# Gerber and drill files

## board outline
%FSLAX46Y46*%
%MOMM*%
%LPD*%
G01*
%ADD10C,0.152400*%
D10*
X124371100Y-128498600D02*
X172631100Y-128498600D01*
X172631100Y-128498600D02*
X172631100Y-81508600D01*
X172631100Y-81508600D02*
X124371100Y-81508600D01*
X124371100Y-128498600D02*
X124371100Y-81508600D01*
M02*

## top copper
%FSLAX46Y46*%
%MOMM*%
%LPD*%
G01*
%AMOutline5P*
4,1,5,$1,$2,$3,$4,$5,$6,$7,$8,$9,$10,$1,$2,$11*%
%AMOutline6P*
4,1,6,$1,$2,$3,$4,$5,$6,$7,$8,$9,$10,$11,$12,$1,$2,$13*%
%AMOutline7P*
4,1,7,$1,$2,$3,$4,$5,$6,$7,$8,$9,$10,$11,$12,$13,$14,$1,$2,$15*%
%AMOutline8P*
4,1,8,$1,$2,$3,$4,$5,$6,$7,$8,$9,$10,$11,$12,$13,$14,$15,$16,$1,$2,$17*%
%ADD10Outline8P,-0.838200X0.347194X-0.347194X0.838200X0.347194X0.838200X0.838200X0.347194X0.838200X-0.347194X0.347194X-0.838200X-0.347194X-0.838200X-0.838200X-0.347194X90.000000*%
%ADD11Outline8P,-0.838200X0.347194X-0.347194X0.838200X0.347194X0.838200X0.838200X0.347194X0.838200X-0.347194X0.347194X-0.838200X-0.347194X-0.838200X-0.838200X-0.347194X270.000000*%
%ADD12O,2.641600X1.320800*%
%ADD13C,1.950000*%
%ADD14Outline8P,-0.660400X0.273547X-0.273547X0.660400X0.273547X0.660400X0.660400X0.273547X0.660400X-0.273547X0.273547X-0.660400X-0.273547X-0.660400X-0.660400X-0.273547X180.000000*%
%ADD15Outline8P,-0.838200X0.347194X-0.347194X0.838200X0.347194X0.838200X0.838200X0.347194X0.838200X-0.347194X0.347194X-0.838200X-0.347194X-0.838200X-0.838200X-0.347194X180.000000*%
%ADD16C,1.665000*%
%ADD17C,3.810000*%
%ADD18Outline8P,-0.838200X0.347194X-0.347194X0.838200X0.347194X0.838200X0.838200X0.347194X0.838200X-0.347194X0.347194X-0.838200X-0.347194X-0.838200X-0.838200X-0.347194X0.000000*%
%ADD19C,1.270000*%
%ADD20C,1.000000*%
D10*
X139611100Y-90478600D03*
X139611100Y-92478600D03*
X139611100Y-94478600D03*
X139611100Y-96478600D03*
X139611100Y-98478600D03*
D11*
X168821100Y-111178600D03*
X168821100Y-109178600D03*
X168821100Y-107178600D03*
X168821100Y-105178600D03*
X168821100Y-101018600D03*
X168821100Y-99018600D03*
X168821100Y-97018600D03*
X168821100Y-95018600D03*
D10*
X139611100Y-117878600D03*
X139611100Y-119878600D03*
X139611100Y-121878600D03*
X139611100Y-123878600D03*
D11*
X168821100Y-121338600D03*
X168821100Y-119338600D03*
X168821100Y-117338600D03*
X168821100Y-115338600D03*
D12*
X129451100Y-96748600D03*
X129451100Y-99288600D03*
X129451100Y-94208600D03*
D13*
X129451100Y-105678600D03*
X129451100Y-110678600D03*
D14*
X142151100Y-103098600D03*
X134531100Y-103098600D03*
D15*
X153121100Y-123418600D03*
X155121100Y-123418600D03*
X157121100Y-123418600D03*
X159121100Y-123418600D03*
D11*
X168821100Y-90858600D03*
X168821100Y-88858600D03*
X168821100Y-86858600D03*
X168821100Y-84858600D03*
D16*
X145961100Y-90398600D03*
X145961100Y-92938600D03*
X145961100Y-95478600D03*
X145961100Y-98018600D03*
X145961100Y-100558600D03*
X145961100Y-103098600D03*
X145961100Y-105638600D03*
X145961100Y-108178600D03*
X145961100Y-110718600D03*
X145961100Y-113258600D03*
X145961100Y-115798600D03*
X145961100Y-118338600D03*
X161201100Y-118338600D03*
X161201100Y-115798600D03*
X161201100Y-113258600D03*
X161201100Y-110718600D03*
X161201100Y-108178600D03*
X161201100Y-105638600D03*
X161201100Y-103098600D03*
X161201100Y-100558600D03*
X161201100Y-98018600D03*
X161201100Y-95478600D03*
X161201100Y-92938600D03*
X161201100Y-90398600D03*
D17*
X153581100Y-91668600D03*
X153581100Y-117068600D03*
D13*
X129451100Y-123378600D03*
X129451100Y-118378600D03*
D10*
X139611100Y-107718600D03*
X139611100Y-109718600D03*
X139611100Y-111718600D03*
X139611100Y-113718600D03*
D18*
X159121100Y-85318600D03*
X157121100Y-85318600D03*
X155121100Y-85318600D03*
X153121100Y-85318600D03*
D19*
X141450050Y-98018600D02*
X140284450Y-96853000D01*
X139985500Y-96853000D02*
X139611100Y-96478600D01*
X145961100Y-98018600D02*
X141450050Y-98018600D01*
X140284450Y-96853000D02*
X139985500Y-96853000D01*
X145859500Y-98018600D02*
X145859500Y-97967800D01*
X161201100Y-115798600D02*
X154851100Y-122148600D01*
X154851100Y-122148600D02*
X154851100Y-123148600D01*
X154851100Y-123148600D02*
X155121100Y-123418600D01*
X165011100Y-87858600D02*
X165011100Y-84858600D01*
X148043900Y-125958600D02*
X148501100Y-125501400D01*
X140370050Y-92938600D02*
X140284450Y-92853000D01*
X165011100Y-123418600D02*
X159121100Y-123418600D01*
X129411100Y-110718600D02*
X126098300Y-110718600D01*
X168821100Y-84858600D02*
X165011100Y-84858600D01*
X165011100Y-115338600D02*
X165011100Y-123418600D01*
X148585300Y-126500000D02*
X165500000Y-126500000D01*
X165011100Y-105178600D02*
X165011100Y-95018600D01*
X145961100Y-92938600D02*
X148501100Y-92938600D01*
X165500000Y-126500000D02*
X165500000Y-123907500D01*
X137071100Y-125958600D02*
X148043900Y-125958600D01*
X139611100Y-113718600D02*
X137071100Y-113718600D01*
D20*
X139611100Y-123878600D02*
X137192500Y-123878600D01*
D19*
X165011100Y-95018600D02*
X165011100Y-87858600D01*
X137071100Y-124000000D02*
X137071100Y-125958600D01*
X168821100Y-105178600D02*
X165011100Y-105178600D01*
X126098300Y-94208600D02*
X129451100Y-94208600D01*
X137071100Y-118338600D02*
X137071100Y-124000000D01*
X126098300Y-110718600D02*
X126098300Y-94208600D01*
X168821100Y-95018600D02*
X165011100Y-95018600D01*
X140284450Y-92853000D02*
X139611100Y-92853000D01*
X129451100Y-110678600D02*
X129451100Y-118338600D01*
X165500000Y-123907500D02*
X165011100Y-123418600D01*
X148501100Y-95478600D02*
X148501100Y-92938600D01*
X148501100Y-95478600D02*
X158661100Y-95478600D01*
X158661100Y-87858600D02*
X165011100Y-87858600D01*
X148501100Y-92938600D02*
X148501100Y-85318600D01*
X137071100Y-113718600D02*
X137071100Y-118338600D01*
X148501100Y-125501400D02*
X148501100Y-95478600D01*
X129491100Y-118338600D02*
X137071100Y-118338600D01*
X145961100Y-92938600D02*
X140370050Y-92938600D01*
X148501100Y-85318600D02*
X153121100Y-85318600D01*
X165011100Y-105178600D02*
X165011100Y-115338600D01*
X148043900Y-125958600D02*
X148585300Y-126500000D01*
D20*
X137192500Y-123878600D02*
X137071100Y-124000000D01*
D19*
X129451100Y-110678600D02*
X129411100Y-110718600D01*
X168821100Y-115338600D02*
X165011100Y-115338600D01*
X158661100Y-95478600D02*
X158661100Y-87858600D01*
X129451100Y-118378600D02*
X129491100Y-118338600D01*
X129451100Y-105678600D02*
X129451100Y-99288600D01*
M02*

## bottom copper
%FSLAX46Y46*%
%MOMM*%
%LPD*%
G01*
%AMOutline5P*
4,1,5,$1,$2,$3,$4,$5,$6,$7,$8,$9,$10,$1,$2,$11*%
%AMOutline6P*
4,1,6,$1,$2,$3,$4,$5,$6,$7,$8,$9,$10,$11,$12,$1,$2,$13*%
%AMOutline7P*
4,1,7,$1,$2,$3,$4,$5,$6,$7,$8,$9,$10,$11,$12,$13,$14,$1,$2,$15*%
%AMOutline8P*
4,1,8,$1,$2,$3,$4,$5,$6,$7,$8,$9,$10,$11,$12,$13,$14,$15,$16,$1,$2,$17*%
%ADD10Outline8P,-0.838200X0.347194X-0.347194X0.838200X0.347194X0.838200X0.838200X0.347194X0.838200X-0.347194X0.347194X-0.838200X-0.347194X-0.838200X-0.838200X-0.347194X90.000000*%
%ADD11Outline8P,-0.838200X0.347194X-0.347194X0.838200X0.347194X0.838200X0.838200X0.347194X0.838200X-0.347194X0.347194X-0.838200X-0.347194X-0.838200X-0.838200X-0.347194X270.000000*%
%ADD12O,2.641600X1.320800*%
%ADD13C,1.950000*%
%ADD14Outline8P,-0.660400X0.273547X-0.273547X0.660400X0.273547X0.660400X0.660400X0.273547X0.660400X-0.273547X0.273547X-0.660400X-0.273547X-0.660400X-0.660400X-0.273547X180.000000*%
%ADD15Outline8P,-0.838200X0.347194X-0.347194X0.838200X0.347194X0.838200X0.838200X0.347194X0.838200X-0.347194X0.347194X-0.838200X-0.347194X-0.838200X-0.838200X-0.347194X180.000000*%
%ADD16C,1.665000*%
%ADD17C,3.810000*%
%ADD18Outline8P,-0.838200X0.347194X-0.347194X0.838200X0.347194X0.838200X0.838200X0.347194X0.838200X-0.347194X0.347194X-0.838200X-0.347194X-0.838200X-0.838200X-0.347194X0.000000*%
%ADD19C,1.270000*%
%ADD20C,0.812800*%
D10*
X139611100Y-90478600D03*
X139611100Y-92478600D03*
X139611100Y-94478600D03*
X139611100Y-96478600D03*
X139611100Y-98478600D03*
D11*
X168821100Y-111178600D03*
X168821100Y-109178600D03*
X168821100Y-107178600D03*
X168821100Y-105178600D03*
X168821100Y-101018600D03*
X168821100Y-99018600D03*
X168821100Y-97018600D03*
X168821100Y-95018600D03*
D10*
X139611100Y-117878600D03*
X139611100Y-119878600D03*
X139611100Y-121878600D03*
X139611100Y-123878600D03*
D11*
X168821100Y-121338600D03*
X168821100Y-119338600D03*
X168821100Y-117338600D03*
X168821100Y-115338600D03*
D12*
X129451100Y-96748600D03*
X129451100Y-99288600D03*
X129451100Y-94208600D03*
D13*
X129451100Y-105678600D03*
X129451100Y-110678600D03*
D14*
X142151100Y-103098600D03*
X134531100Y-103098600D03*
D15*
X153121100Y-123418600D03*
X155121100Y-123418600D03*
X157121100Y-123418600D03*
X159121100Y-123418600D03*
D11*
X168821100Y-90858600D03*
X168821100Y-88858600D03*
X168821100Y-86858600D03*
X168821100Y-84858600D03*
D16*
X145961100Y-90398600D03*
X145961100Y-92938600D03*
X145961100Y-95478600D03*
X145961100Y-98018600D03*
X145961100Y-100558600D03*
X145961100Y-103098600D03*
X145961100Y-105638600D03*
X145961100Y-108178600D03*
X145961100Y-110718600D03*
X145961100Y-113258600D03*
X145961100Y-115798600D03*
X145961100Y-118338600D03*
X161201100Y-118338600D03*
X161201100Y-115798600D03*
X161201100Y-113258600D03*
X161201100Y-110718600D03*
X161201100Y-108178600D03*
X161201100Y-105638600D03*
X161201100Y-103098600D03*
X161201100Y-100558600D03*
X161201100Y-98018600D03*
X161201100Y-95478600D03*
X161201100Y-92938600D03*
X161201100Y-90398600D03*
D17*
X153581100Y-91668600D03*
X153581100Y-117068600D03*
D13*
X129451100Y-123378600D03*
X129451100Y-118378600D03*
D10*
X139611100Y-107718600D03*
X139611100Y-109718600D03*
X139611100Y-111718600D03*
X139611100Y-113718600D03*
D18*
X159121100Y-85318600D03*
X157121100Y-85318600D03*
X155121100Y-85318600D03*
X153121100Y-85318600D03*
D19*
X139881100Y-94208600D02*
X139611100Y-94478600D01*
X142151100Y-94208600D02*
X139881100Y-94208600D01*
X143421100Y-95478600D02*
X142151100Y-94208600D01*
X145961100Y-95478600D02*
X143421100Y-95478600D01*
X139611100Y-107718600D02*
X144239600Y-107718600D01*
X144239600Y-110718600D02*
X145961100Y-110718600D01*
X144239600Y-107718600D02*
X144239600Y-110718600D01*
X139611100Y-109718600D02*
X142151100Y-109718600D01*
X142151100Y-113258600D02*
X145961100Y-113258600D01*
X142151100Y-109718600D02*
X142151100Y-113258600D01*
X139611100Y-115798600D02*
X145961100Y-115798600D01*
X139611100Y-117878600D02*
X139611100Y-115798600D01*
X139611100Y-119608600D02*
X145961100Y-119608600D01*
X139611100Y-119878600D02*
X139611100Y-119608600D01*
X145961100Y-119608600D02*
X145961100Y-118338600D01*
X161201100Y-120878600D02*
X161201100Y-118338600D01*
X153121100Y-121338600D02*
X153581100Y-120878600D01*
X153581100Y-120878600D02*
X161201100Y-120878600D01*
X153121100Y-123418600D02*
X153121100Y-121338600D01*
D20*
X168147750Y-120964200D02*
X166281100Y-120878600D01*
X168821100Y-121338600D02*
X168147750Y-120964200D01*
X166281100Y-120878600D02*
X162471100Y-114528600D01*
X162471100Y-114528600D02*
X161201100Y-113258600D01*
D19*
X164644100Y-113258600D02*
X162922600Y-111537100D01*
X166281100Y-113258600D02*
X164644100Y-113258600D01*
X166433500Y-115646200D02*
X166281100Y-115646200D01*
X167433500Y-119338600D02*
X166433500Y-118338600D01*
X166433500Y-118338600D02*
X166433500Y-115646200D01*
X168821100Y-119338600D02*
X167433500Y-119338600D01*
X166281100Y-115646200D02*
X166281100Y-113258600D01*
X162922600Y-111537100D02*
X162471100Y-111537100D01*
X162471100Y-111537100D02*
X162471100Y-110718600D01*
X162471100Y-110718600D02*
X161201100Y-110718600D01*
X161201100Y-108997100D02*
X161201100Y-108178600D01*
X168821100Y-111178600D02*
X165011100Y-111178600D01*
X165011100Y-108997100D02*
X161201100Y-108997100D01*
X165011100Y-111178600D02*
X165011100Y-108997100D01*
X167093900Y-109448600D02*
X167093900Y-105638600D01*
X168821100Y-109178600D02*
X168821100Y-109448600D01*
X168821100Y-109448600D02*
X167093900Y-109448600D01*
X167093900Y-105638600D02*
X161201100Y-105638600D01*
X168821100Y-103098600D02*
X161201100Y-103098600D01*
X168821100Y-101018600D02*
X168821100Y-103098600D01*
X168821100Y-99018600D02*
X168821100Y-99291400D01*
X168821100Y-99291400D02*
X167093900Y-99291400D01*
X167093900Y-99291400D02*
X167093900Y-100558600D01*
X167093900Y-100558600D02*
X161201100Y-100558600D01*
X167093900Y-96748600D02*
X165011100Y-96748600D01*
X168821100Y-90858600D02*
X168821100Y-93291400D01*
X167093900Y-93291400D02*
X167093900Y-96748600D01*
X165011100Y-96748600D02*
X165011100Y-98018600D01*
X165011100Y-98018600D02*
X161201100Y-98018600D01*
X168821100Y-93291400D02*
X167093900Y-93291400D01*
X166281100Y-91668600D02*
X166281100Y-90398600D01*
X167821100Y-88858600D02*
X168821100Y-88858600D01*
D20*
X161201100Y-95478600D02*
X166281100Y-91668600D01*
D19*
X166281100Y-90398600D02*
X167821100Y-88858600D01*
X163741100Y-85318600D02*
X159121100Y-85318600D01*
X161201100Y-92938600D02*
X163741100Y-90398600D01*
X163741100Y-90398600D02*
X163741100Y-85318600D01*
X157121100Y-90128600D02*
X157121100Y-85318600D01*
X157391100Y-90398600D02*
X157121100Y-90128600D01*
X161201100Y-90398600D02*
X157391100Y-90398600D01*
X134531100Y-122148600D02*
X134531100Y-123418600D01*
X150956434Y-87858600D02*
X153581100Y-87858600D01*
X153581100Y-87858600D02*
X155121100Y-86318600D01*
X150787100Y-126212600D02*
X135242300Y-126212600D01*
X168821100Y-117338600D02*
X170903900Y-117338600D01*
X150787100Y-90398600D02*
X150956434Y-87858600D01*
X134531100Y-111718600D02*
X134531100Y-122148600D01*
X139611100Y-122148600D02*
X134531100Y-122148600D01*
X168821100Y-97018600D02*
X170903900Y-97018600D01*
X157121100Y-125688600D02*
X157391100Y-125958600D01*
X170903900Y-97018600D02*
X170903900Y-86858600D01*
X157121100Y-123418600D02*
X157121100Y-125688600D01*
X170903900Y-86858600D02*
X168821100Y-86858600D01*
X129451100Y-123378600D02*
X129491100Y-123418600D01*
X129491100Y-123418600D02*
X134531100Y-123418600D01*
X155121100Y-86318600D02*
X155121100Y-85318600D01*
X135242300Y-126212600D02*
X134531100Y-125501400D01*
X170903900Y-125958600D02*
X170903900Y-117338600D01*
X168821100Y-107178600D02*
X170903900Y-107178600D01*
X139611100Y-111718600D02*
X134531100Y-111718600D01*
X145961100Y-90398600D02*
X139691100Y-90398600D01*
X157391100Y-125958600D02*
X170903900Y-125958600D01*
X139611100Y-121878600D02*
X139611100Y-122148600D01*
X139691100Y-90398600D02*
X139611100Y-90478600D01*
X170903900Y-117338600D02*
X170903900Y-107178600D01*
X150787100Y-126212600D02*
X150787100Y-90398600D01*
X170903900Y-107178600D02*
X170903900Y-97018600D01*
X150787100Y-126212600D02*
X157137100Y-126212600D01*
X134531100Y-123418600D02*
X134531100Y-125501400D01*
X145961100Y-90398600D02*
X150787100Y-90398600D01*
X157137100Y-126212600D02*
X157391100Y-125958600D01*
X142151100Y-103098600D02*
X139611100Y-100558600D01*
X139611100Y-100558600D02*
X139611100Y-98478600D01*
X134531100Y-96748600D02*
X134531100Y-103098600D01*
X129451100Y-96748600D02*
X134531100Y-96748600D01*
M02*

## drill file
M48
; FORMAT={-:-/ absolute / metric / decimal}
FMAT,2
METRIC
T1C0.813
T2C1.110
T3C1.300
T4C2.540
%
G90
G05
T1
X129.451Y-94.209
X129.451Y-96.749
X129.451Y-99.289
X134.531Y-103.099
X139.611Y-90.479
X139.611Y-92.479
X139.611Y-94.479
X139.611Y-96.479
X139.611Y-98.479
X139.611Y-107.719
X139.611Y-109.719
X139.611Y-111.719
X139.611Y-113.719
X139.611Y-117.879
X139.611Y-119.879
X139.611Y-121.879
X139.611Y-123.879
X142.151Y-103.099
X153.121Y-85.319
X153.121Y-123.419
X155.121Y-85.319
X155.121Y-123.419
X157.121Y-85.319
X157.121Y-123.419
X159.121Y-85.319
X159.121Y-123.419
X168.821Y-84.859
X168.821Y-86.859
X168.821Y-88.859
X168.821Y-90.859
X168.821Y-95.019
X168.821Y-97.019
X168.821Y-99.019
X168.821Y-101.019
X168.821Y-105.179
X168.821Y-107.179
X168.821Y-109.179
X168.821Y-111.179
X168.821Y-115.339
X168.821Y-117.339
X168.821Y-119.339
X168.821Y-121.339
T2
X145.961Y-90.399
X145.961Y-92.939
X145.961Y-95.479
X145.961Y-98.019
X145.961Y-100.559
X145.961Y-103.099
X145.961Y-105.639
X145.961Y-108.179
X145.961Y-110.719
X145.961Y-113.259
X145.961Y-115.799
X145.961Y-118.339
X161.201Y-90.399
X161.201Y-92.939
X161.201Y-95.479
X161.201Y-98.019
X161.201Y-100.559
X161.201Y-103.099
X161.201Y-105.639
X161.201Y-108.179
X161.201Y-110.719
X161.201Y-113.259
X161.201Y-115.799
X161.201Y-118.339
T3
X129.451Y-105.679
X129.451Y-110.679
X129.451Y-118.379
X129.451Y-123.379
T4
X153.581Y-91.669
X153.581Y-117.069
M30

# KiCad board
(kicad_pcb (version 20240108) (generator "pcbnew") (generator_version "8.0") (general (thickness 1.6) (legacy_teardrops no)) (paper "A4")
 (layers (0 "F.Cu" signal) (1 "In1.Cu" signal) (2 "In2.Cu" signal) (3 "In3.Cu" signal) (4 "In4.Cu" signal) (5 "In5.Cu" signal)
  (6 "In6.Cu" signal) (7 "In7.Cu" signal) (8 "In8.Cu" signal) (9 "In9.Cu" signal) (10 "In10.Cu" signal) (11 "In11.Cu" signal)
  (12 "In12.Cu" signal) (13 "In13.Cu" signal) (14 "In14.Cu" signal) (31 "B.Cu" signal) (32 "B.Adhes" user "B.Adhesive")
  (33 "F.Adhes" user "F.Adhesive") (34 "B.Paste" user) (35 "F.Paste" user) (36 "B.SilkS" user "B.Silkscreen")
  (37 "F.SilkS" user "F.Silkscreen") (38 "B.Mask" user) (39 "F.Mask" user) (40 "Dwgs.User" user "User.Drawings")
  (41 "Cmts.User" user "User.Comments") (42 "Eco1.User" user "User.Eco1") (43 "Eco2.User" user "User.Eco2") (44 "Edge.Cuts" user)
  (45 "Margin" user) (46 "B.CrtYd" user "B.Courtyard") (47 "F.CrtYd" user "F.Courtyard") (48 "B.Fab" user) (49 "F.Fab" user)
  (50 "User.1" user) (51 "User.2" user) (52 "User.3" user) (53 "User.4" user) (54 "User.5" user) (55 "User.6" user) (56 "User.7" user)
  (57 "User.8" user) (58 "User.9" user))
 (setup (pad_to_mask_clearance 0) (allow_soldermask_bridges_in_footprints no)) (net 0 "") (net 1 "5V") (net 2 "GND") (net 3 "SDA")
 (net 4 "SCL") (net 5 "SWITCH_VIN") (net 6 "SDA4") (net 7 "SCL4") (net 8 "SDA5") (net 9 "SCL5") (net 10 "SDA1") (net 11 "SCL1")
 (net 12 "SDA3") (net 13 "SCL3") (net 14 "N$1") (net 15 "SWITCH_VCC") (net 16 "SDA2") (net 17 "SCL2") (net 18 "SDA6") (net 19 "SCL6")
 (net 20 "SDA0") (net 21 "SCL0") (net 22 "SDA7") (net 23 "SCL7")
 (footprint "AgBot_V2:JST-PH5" (layer "F.Cu") (at 139.6111 95.4786 90)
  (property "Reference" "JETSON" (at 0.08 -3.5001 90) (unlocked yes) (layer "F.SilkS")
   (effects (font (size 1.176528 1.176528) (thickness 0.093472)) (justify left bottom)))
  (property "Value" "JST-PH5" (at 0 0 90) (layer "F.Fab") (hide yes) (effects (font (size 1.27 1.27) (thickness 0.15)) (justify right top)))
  (pad "1" thru_hole roundrect (at 5 0 90) (size 1.6764 1.6764) (drill 0.8128) (layers "*.Cu" "*.Mask") (remove_unused_layers no)
   (roundrect_rratio 0.25) (chamfer_ratio 0.2928932188) (chamfer top_left top_right bottom_left bottom_right) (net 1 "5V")
   (solder_mask_margin 0.1016) (thermal_bridge_angle 0))
  (pad "2" thru_hole roundrect (at 3 0 90) (size 1.6764 1.6764) (drill 0.8128) (layers "*.Cu" "*.Mask") (remove_unused_layers no)
   (roundrect_rratio 0.25) (chamfer_ratio 0.2928932188) (chamfer top_left top_right bottom_left bottom_right) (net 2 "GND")
   (solder_mask_margin 0.1016) (thermal_bridge_angle 0))
  (pad "3" thru_hole roundrect (at 1 0 90) (size 1.6764 1.6764) (drill 0.8128) (layers "*.Cu" "*.Mask") (remove_unused_layers no)
   (roundrect_rratio 0.25) (chamfer_ratio 0.2928932188) (chamfer top_left top_right bottom_left bottom_right) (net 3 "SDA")
   (solder_mask_margin 0.1016) (thermal_bridge_angle 0))
  (pad "4" thru_hole roundrect (at -1 0 90) (size 1.6764 1.6764) (drill 0.8128) (layers "*.Cu" "*.Mask") (remove_unused_layers no)
   (roundrect_rratio 0.25) (chamfer_ratio 0.2928932188) (chamfer top_left top_right bottom_left bottom_right) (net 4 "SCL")
   (solder_mask_margin 0.1016) (thermal_bridge_angle 0))
  (pad "5" thru_hole roundrect (at -3 0 90) (size 1.6764 1.6764) (drill 0.8128) (layers "*.Cu" "*.Mask") (remove_unused_layers no)
   (roundrect_rratio 0.25) (chamfer_ratio 0.2928932188) (chamfer top_left top_right bottom_left bottom_right) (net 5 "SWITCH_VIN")
   (solder_mask_margin 0.1016) (thermal_bridge_angle 0)))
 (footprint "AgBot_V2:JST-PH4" (layer "F.Cu") (at 168.8211 108.1786 -90)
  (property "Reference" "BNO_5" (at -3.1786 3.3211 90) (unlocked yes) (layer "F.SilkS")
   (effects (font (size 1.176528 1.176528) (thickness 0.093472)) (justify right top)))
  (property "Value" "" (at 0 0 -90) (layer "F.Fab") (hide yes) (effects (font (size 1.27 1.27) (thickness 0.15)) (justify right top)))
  (pad "1" thru_hole roundrect (at 3 0 270) (size 1.6764 1.6764) (drill 0.8128) (layers "*.Cu" "*.Mask") (remove_unused_layers no)
   (roundrect_rratio 0.25) (chamfer_ratio 0.2928932188) (chamfer top_left top_right bottom_left bottom_right) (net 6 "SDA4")
   (solder_mask_margin 0.1016) (thermal_bridge_angle 0))
  (pad "2" thru_hole roundrect (at 1 0 270) (size 1.6764 1.6764) (drill 0.8128) (layers "*.Cu" "*.Mask") (remove_unused_layers no)
   (roundrect_rratio 0.25) (chamfer_ratio 0.2928932188) (chamfer top_left top_right bottom_left bottom_right) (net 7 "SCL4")
   (solder_mask_margin 0.1016) (thermal_bridge_angle 0))
  (pad "3" thru_hole roundrect (at -1 0 270) (size 1.6764 1.6764) (drill 0.8128) (layers "*.Cu" "*.Mask") (remove_unused_layers no)
   (roundrect_rratio 0.25) (chamfer_ratio 0.2928932188) (chamfer top_left top_right bottom_left bottom_right) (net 1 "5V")
   (solder_mask_margin 0.1016) (thermal_bridge_angle 0))
  (pad "4" thru_hole roundrect (at -3 0 270) (size 1.6764 1.6764) (drill 0.8128) (layers "*.Cu" "*.Mask") (remove_unused_layers no)
   (roundrect_rratio 0.25) (chamfer_ratio 0.2928932188) (chamfer top_left top_right bottom_left bottom_right) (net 2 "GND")
   (solder_mask_margin 0.1016) (thermal_bridge_angle 0)))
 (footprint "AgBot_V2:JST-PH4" (layer "F.Cu") (at 168.8211 98.0186 -90)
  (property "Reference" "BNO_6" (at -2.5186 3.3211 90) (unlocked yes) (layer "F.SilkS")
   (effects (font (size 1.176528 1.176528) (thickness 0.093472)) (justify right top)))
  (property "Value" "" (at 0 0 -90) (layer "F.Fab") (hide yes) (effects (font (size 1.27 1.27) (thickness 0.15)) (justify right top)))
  (pad "1" thru_hole roundrect (at 3 0 270) (size 1.6764 1.6764) (drill 0.8128) (layers "*.Cu" "*.Mask") (remove_unused_layers no)
   (roundrect_rratio 0.25) (chamfer_ratio 0.2928932188) (chamfer top_left top_right bottom_left bottom_right) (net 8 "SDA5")
   (solder_mask_margin 0.1016) (thermal_bridge_angle 0))
  (pad "2" thru_hole roundrect (at 1 0 270) (size 1.6764 1.6764) (drill 0.8128) (layers "*.Cu" "*.Mask") (remove_unused_layers no)
   (roundrect_rratio 0.25) (chamfer_ratio 0.2928932188) (chamfer top_left top_right bottom_left bottom_right) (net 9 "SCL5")
   (solder_mask_margin 0.1016) (thermal_bridge_angle 0))
  (pad "3" thru_hole roundrect (at -1 0 270) (size 1.6764 1.6764) (drill 0.8128) (layers "*.Cu" "*.Mask") (remove_unused_layers no)
   (roundrect_rratio 0.25) (chamfer_ratio 0.2928932188) (chamfer top_left top_right bottom_left bottom_right) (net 1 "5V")
   (solder_mask_margin 0.1016) (thermal_bridge_angle 0))
  (pad "4" thru_hole roundrect (at -3 0 270) (size 1.6764 1.6764) (drill 0.8128) (layers "*.Cu" "*.Mask") (remove_unused_layers no)
   (roundrect_rratio 0.25) (chamfer_ratio 0.2928932188) (chamfer top_left top_right bottom_left bottom_right) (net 2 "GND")
   (solder_mask_margin 0.1016) (thermal_bridge_angle 0)))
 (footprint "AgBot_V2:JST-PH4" (layer "F.Cu") (at 139.6111 120.8786 90)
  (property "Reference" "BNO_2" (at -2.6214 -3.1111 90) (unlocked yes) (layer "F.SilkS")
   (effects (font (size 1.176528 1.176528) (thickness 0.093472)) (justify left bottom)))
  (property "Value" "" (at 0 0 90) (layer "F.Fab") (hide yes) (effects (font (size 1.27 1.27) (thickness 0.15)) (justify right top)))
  (pad "1" thru_hole roundrect (at 3 0 90) (size 1.6764 1.6764) (drill 0.8128) (layers "*.Cu" "*.Mask") (remove_unused_layers no)
   (roundrect_rratio 0.25) (chamfer_ratio 0.2928932188) (chamfer top_left top_right bottom_left bottom_right) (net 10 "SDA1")
   (solder_mask_margin 0.1016) (thermal_bridge_angle 0))
  (pad "2" thru_hole roundrect (at 1 0 90) (size 1.6764 1.6764) (drill 0.8128) (layers "*.Cu" "*.Mask") (remove_unused_layers no)
   (roundrect_rratio 0.25) (chamfer_ratio 0.2928932188) (chamfer top_left top_right bottom_left bottom_right) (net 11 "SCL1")
   (solder_mask_margin 0.1016) (thermal_bridge_angle 0))
  (pad "3" thru_hole roundrect (at -1 0 90) (size 1.6764 1.6764) (drill 0.8128) (layers "*.Cu" "*.Mask") (remove_unused_layers no)
   (roundrect_rratio 0.25) (chamfer_ratio 0.2928932188) (chamfer top_left top_right bottom_left bottom_right) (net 1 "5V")
   (solder_mask_margin 0.1016) (thermal_bridge_angle 0))
  (pad "4" thru_hole roundrect (at -3 0 90) (size 1.6764 1.6764) (drill 0.8128) (layers "*.Cu" "*.Mask") (remove_unused_layers no)
   (roundrect_rratio 0.25) (chamfer_ratio 0.2928932188) (chamfer top_left top_right bottom_left bottom_right) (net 2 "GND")
   (solder_mask_margin 0.1016) (thermal_bridge_angle 0)))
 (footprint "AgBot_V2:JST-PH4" (layer "F.Cu") (at 168.8211 118.3386 -90)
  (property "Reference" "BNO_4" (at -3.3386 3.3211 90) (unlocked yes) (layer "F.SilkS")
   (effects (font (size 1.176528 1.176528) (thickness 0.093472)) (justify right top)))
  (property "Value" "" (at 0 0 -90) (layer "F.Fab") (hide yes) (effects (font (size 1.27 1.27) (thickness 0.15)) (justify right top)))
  (pad "1" thru_hole roundrect (at 3 0 270) (size 1.6764 1.6764) (drill 0.8128) (layers "*.Cu" "*.Mask") (remove_unused_layers no)
   (roundrect_rratio 0.25) (chamfer_ratio 0.2928932188) (chamfer top_left top_right bottom_left bottom_right) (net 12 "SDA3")
   (solder_mask_margin 0.1016) (thermal_bridge_angle 0))
  (pad "2" thru_hole roundrect (at 1 0 270) (size 1.6764 1.6764) (drill 0.8128) (layers "*.Cu" "*.Mask") (remove_unused_layers no)
   (roundrect_rratio 0.25) (chamfer_ratio 0.2928932188) (chamfer top_left top_right bottom_left bottom_right) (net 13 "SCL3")
   (solder_mask_margin 0.1016) (thermal_bridge_angle 0))
  (pad "3" thru_hole roundrect (at -1 0 270) (size 1.6764 1.6764) (drill 0.8128) (layers "*.Cu" "*.Mask") (remove_unused_layers no)
   (roundrect_rratio 0.25) (chamfer_ratio 0.2928932188) (chamfer top_left top_right bottom_left bottom_right) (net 1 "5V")
   (solder_mask_margin 0.1016) (thermal_bridge_angle 0))
  (pad "4" thru_hole roundrect (at -3 0 270) (size 1.6764 1.6764) (drill 0.8128) (layers "*.Cu" "*.Mask") (remove_unused_layers no)
   (roundrect_rratio 0.25) (chamfer_ratio 0.2928932188) (chamfer top_left top_right bottom_left bottom_right) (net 2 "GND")
   (solder_mask_margin 0.1016) (thermal_bridge_angle 0)))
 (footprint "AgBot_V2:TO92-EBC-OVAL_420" (layer "F.Cu") (at 130.7211 96.7486 -90)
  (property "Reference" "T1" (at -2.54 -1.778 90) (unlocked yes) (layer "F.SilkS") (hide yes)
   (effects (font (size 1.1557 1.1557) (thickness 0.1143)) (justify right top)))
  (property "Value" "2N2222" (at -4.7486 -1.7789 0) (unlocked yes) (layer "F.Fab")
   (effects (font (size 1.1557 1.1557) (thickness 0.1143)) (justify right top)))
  (pad "B" thru_hole oval (at 0 1.27) (size 2.6416 1.3208) (drill 0.8128) (layers "*.Cu" "*.Mask") (remove_unused_layers no) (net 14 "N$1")
   (solder_mask_margin 0.1016) (thermal_bridge_angle 0))
  (pad "C" thru_hole oval (at 2.54 1.27) (size 2.6416 1.3208) (drill 0.8128) (layers "*.Cu" "*.Mask") (remove_unused_layers no)
   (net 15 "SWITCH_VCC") (solder_mask_margin 0.1016) (thermal_bridge_angle 0))
  (pad "E" thru_hole oval (at -2.54 1.27) (size 2.6416 1.3208) (drill 0.8128) (layers "*.Cu" "*.Mask") (remove_unused_layers no)
   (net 2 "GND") (solder_mask_margin 0.1016) (thermal_bridge_angle 0)))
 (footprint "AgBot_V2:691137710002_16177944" (layer "F.Cu") (at 129.4511 108.1786 -90)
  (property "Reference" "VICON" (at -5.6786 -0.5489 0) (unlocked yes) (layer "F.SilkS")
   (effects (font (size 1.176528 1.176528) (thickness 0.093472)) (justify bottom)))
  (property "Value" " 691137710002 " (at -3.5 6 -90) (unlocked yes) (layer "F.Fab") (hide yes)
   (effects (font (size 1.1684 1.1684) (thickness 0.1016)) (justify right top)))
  (pad "1" thru_hole circle (at -2.5 0 270) (size 1.95 1.95) (drill 1.3) (layers "*.Cu" "*.Mask") (remove_unused_layers no)
   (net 15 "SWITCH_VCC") (solder_mask_margin 0.1016) (thermal_bridge_angle 0))
  (pad "2" thru_hole circle (at 2.5 0 270) (size 1.95 1.95) (drill 1.3) (layers "*.Cu" "*.Mask") (remove_unused_layers no) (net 2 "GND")
   (solder_mask_margin 0.1016) (thermal_bridge_angle 0)))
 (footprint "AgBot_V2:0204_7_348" (layer "F.Cu") (at 138.3411 103.0986 180)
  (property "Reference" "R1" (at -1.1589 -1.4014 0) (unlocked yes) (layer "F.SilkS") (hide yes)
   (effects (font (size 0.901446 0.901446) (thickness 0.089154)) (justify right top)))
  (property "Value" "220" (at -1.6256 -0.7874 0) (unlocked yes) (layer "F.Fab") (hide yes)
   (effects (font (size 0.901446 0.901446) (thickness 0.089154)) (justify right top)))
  (pad "1" thru_hole roundrect (at -3.81 0 180) (size 1.3208 1.3208) (drill 0.8128) (layers "*.Cu" "*.Mask") (remove_unused_layers no)
   (roundrect_rratio 0.25) (chamfer_ratio 0.2928932188) (chamfer top_left top_right bottom_left bottom_right) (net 5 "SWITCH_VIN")
   (solder_mask_margin 0.1016) (thermal_bridge_angle 0))
  (pad "2" thru_hole roundrect (at 3.81 0 180) (size 1.3208 1.3208) (drill 0.8128) (layers "*.Cu" "*.Mask") (remove_unused_layers no)
   (roundrect_rratio 0.25) (chamfer_ratio 0.2928932188) (chamfer top_left top_right bottom_left bottom_right) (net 14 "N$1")
   (solder_mask_margin 0.1016) (thermal_bridge_angle 0)))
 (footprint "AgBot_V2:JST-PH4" (layer "F.Cu") (at 156.1211 123.4186 180)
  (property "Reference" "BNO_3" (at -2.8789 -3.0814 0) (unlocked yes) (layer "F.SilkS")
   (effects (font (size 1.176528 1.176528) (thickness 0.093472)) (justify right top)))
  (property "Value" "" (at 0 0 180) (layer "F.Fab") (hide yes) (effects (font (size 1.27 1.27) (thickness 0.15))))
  (pad "1" thru_hole roundrect (at 3 0 180) (size 1.6764 1.6764) (drill 0.8128) (layers "*.Cu" "*.Mask") (remove_unused_layers no)
   (roundrect_rratio 0.25) (chamfer_ratio 0.2928932188) (chamfer top_left top_right bottom_left bottom_right) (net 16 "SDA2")
   (solder_mask_margin 0.1016) (thermal_bridge_angle 0))
  (pad "2" thru_hole roundrect (at 1 0 180) (size 1.6764 1.6764) (drill 0.8128) (layers "*.Cu" "*.Mask") (remove_unused_layers no)
   (roundrect_rratio 0.25) (chamfer_ratio 0.2928932188) (chamfer top_left top_right bottom_left bottom_right) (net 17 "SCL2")
   (solder_mask_margin 0.1016) (thermal_bridge_angle 0))
  (pad "3" thru_hole roundrect (at -1 0 180) (size 1.6764 1.6764) (drill 0.8128) (layers "*.Cu" "*.Mask") (remove_unused_layers no)
   (roundrect_rratio 0.25) (chamfer_ratio 0.2928932188) (chamfer top_left top_right bottom_left bottom_right) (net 1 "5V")
   (solder_mask_margin 0.1016) (thermal_bridge_angle 0))
  (pad "4" thru_hole roundrect (at -3 0 180) (size 1.6764 1.6764) (drill 0.8128) (layers "*.Cu" "*.Mask") (remove_unused_layers no)
   (roundrect_rratio 0.25) (chamfer_ratio 0.2928932188) (chamfer top_left top_right bottom_left bottom_right) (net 2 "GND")
   (solder_mask_margin 0.1016) (thermal_bridge_angle 0)))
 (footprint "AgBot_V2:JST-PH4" (layer "F.Cu") (at 168.8211 87.8586 -90)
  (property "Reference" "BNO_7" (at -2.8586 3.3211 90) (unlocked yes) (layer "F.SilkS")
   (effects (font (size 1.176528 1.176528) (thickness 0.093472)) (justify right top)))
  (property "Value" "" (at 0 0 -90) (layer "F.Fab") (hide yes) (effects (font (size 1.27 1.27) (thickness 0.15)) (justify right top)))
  (pad "1" thru_hole roundrect (at 3 0 270) (size 1.6764 1.6764) (drill 0.8128) (layers "*.Cu" "*.Mask") (remove_unused_layers no)
   (roundrect_rratio 0.25) (chamfer_ratio 0.2928932188) (chamfer top_left top_right bottom_left bottom_right) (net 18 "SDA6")
   (solder_mask_margin 0.1016) (thermal_bridge_angle 0))
  (pad "2" thru_hole roundrect (at 1 0 270) (size 1.6764 1.6764) (drill 0.8128) (layers "*.Cu" "*.Mask") (remove_unused_layers no)
   (roundrect_rratio 0.25) (chamfer_ratio 0.2928932188) (chamfer top_left top_right bottom_left bottom_right) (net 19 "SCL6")
   (solder_mask_margin 0.1016) (thermal_bridge_angle 0))
  (pad "3" thru_hole roundrect (at -1 0 270) (size 1.6764 1.6764) (drill 0.8128) (layers "*.Cu" "*.Mask") (remove_unused_layers no)
   (roundrect_rratio 0.25) (chamfer_ratio 0.2928932188) (chamfer top_left top_right bottom_left bottom_right) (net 1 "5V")
   (solder_mask_margin 0.1016) (thermal_bridge_angle 0))
  (pad "4" thru_hole roundrect (at -3 0 270) (size 1.6764 1.6764) (drill 0.8128) (layers "*.Cu" "*.Mask") (remove_unused_layers no)
   (roundrect_rratio 0.25) (chamfer_ratio 0.2928932188) (chamfer top_left top_right bottom_left bottom_right) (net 2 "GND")
   (solder_mask_margin 0.1016) (thermal_bridge_angle 0)))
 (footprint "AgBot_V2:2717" (layer "F.Cu") (at 153.5811 104.3686)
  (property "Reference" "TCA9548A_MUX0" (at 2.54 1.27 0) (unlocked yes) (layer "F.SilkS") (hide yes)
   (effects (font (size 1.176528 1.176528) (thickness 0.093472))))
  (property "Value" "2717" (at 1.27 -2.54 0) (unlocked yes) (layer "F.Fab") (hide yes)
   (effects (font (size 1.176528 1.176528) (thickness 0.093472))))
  (pad "1" thru_hole circle (at -7.62 -13.97) (size 1.665 1.665) (drill 1.11) (layers "*.Cu" "*.Mask") (remove_unused_layers no)
   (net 1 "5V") (solder_mask_margin 0.1016) (thermal_bridge_angle 0))
  (pad "2" thru_hole circle (at -7.62 -11.43) (size 1.665 1.665) (drill 1.11) (layers "*.Cu" "*.Mask") (remove_unused_layers no)
   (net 2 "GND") (solder_mask_margin 0.1016) (thermal_bridge_angle 0))
  (pad "3" thru_hole circle (at -7.62 -8.89) (size 1.665 1.665) (drill 1.11) (layers "*.Cu" "*.Mask") (remove_unused_layers no)
   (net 3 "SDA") (solder_mask_margin 0.1016) (thermal_bridge_angle 0))
  (pad "4" thru_hole circle (at -7.62 -6.35) (size 1.665 1.665) (drill 1.11) (layers "*.Cu" "*.Mask") (remove_unused_layers no)
   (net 4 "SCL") (solder_mask_margin 0.1016) (thermal_bridge_angle 0))
  (pad "5" thru_hole circle (at -7.62 -3.81) (size 1.665 1.665) (drill 1.11) (layers "*.Cu" "*.Mask") (remove_unused_layers no)
   (solder_mask_margin 0.1016) (thermal_bridge_angle 0))
  (pad "6" thru_hole circle (at -7.62 -1.27) (size 1.665 1.665) (drill 1.11) (layers "*.Cu" "*.Mask") (remove_unused_layers no)
   (solder_mask_margin 0.1016) (thermal_bridge_angle 0))
  (pad "7" thru_hole circle (at -7.62 1.27) (size 1.665 1.665) (drill 1.11) (layers "*.Cu" "*.Mask") (remove_unused_layers no)
   (solder_mask_margin 0.1016) (thermal_bridge_angle 0))
  (pad "8" thru_hole circle (at -7.62 3.81) (size 1.665 1.665) (drill 1.11) (layers "*.Cu" "*.Mask") (remove_unused_layers no)
   (solder_mask_margin 0.1016) (thermal_bridge_angle 0))
  (pad "9" thru_hole circle (at -7.62 6.35) (size 1.665 1.665) (drill 1.11) (layers "*.Cu" "*.Mask") (remove_unused_layers no)
   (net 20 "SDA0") (solder_mask_margin 0.1016) (thermal_bridge_angle 0))
  (pad "10" thru_hole circle (at -7.62 8.89) (size 1.665 1.665) (drill 1.11) (layers "*.Cu" "*.Mask") (remove_unused_layers no)
   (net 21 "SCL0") (solder_mask_margin 0.1016) (thermal_bridge_angle 0))
  (pad "11" thru_hole circle (at -7.62 11.43) (size 1.665 1.665) (drill 1.11) (layers "*.Cu" "*.Mask") (remove_unused_layers no)
   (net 10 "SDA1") (solder_mask_margin 0.1016) (thermal_bridge_angle 0))
  (pad "12" thru_hole circle (at -7.62 13.97) (size 1.665 1.665) (drill 1.11) (layers "*.Cu" "*.Mask") (remove_unused_layers no)
   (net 11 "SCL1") (solder_mask_margin 0.1016) (thermal_bridge_angle 0))
  (pad "13" thru_hole circle (at 7.62 13.97) (size 1.665 1.665) (drill 1.11) (layers "*.Cu" "*.Mask") (remove_unused_layers no)
   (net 16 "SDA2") (solder_mask_margin 0.1016) (thermal_bridge_angle 0))
  (pad "14" thru_hole circle (at 7.62 11.43) (size 1.665 1.665) (drill 1.11) (layers "*.Cu" "*.Mask") (remove_unused_layers no)
   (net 17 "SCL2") (solder_mask_margin 0.1016) (thermal_bridge_angle 0))
  (pad "15" thru_hole circle (at 7.62 8.89) (size 1.665 1.665) (drill 1.11) (layers "*.Cu" "*.Mask") (remove_unused_layers no)
   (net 12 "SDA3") (solder_mask_margin 0.1016) (thermal_bridge_angle 0))
  (pad "16" thru_hole circle (at 7.62 6.35) (size 1.665 1.665) (drill 1.11) (layers "*.Cu" "*.Mask") (remove_unused_layers no)
   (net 13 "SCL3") (solder_mask_margin 0.1016) (thermal_bridge_angle 0))
  (pad "17" thru_hole circle (at 7.62 3.81) (size 1.665 1.665) (drill 1.11) (layers "*.Cu" "*.Mask") (remove_unused_layers no)
   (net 6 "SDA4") (solder_mask_margin 0.1016) (thermal_bridge_angle 0))
  (pad "18" thru_hole circle (at 7.62 1.27) (size 1.665 1.665) (drill 1.11) (layers "*.Cu" "*.Mask") (remove_unused_layers no)
   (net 7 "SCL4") (solder_mask_margin 0.1016) (thermal_bridge_angle 0))
  (pad "19" thru_hole circle (at 7.62 -1.27) (size 1.665 1.665) (drill 1.11) (layers "*.Cu" "*.Mask") (remove_unused_layers no)
   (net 8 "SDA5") (solder_mask_margin 0.1016) (thermal_bridge_angle 0))
  (pad "20" thru_hole circle (at 7.62 -3.81) (size 1.665 1.665) (drill 1.11) (layers "*.Cu" "*.Mask") (remove_unused_layers no)
   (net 9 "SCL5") (solder_mask_margin 0.1016) (thermal_bridge_angle 0))
  (pad "21" thru_hole circle (at 7.62 -6.35) (size 1.665 1.665) (drill 1.11) (layers "*.Cu" "*.Mask") (remove_unused_layers no)
   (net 18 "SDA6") (solder_mask_margin 0.1016) (thermal_bridge_angle 0))
  (pad "22" thru_hole circle (at 7.62 -8.89) (size 1.665 1.665) (drill 1.11) (layers "*.Cu" "*.Mask") (remove_unused_layers no)
   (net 19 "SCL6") (solder_mask_margin 0.1016) (thermal_bridge_angle 0))
  (pad "23" thru_hole circle (at 7.62 -11.43) (size 1.665 1.665) (drill 1.11) (layers "*.Cu" "*.Mask") (remove_unused_layers no)
   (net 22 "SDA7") (solder_mask_margin 0.1016) (thermal_bridge_angle 0))
  (pad "24" thru_hole circle (at 7.62 -13.97) (size 1.665 1.665) (drill 1.11) (layers "*.Cu" "*.Mask") (remove_unused_layers no)
   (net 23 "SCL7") (solder_mask_margin 0.1016) (thermal_bridge_angle 0))
  (pad "25" thru_hole circle (at 0 -12.7) (size 3.81 3.81) (drill 2.54) (layers "*.Cu" "*.Mask") (remove_unused_layers no)
   (solder_mask_margin 0.1016) (thermal_bridge_angle 0))
  (pad "26" thru_hole circle (at 0 12.7) (size 3.81 3.81) (drill 2.54) (layers "*.Cu" "*.Mask") (remove_unused_layers no)
   (solder_mask_margin 0.1016) (thermal_bridge_angle 0)))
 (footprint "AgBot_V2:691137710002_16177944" (layer "F.Cu") (at 129.4511 120.8786 90)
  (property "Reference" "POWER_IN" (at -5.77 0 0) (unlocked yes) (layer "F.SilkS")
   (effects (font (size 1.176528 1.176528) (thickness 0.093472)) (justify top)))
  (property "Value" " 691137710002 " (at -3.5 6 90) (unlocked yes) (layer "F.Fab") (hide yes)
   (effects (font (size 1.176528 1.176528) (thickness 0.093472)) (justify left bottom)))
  (pad "1" thru_hole circle (at -2.5 0 90) (size 1.95 1.95) (drill 1.3) (layers "*.Cu" "*.Mask") (remove_unused_layers no) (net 1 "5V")
   (solder_mask_margin 0.1016) (thermal_bridge_angle 0))
  (pad "2" thru_hole circle (at 2.5 0 90) (size 1.95 1.95) (drill 1.3) (layers "*.Cu" "*.Mask") (remove_unused_layers no) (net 2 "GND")
   (solder_mask_margin 0.1016) (thermal_bridge_angle 0)))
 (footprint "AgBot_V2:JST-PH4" (layer "F.Cu") (at 139.6111 110.7186 90)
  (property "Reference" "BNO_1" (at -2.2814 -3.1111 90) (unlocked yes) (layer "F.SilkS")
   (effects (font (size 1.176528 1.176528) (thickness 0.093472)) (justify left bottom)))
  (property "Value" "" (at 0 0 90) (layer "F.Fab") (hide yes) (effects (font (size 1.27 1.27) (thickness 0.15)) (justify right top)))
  (pad "1" thru_hole roundrect (at 3 0 90) (size 1.6764 1.6764) (drill 0.8128) (layers "*.Cu" "*.Mask") (remove_unused_layers no)
   (roundrect_rratio 0.25) (chamfer_ratio 0.2928932188) (chamfer top_left top_right bottom_left bottom_right) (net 20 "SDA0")
   (solder_mask_margin 0.1016) (thermal_bridge_angle 0))
  (pad "2" thru_hole roundrect (at 1 0 90) (size 1.6764 1.6764) (drill 0.8128) (layers "*.Cu" "*.Mask") (remove_unused_layers no)
   (roundrect_rratio 0.25) (chamfer_ratio 0.2928932188) (chamfer top_left top_right bottom_left bottom_right) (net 21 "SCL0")
   (solder_mask_margin 0.1016) (thermal_bridge_angle 0))
  (pad "3" thru_hole roundrect (at -1 0 90) (size 1.6764 1.6764) (drill 0.8128) (layers "*.Cu" "*.Mask") (remove_unused_layers no)
   (roundrect_rratio 0.25) (chamfer_ratio 0.2928932188) (chamfer top_left top_right bottom_left bottom_right) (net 1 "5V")
   (solder_mask_margin 0.1016) (thermal_bridge_angle 0))
  (pad "4" thru_hole roundrect (at -3 0 90) (size 1.6764 1.6764) (drill 0.8128) (layers "*.Cu" "*.Mask") (remove_unused_layers no)
   (roundrect_rratio 0.25) (chamfer_ratio 0.2928932188) (chamfer top_left top_right bottom_left bottom_right) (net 2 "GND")
   (solder_mask_margin 0.1016) (thermal_bridge_angle 0)))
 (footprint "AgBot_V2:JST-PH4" (layer "F.Cu") (at 156.1211 85.3186)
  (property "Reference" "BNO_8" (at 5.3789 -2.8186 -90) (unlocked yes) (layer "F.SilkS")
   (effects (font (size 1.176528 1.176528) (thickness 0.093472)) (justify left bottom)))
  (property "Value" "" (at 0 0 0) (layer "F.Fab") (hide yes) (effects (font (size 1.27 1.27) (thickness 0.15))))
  (pad "1" thru_hole roundrect (at 3 0) (size 1.6764 1.6764) (drill 0.8128) (layers "*.Cu" "*.Mask") (remove_unused_layers no)
   (roundrect_rratio 0.25) (chamfer_ratio 0.2928932188) (chamfer top_left top_right bottom_left bottom_right) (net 22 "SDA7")
   (solder_mask_margin 0.1016) (thermal_bridge_angle 0))
  (pad "2" thru_hole roundrect (at 1 0) (size 1.6764 1.6764) (drill 0.8128) (layers "*.Cu" "*.Mask") (remove_unused_layers no)
   (roundrect_rratio 0.25) (chamfer_ratio 0.2928932188) (chamfer top_left top_right bottom_left bottom_right) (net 23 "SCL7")
   (solder_mask_margin 0.1016) (thermal_bridge_angle 0))
  (pad "3" thru_hole roundrect (at -1 0) (size 1.6764 1.6764) (drill 0.8128) (layers "*.Cu" "*.Mask") (remove_unused_layers no)
   (roundrect_rratio 0.25) (chamfer_ratio 0.2928932188) (chamfer top_left top_right bottom_left bottom_right) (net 1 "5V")
   (solder_mask_margin 0.1016) (thermal_bridge_angle 0))
  (pad "4" thru_hole roundrect (at -3 0) (size 1.6764 1.6764) (drill 0.8128) (layers "*.Cu" "*.Mask") (remove_unused_layers no)
   (roundrect_rratio 0.25) (chamfer_ratio 0.2928932188) (chamfer top_left top_right bottom_left bottom_right) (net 2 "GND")
   (solder_mask_margin 0.1016) (thermal_bridge_angle 0)))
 (gr_line (start 124.3711 128.4986) (end 172.6311 128.4986) (stroke (width 0.1524) (type solid)) (layer "Edge.Cuts"))
 (gr_line (start 172.6311 128.4986) (end 172.6311 81.5086) (stroke (width 0.1524) (type solid)) (layer "Edge.Cuts"))
 (gr_line (start 172.6311 81.5086) (end 124.3711 81.5086) (stroke (width 0.1524) (type solid)) (layer "Edge.Cuts"))
 (gr_line (start 124.3711 128.4986) (end 124.3711 81.5086) (stroke (width 0.1524) (type solid)) (layer "Edge.Cuts"))
 (segment (start 139.8811 94.2086) (end 139.6111 94.4786) (width 1.27) (layer "B.Cu") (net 3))
 (segment (start 142.1511 94.2086) (end 139.8811 94.2086) (width 1.27) (layer "B.Cu") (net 3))
 (segment (start 143.4211 95.4786) (end 142.1511 94.2086) (width 1.27) (layer "B.Cu") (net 3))
 (segment (start 145.9611 95.4786) (end 143.4211 95.4786) (width 1.27) (layer "B.Cu") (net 3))
 (segment (start 141.45005 98.0186) (end 140.28445 96.853) (width 1.27) (layer "F.Cu") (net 4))
 (segment (start 139.9855 96.853) (end 139.6111 96.4786) (width 1.27) (layer "F.Cu") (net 4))
 (segment (start 145.9611 98.0186) (end 141.45005 98.0186) (width 1.27) (layer "F.Cu") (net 4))
 (segment (start 140.28445 96.853) (end 139.9855 96.853) (width 1.27) (layer "F.Cu") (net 4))
 (segment (start 145.8595 98.0186) (end 145.8595 97.9678) (width 1.27) (layer "F.Cu") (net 4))
 (segment (start 139.6111 107.7186) (end 144.2396 107.7186) (width 1.27) (layer "B.Cu") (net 20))
 (segment (start 144.2396 110.7186) (end 145.9611 110.7186) (width 1.27) (layer "B.Cu") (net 20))
 (segment (start 144.2396 107.7186) (end 144.2396 110.7186) (width 1.27) (layer "B.Cu") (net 20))
 (segment (start 139.6111 109.7186) (end 142.1511 109.7186) (width 1.27) (layer "B.Cu") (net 21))
 (segment (start 142.1511 113.2586) (end 145.9611 113.2586) (width 1.27) (layer "B.Cu") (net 21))
 (segment (start 142.1511 109.7186) (end 142.1511 113.2586) (width 1.27) (layer "B.Cu") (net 21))
 (segment (start 139.6111 115.7986) (end 145.9611 115.7986) (width 1.27) (layer "B.Cu") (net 10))
 (segment (start 139.6111 117.8786) (end 139.6111 115.7986) (width 1.27) (layer "B.Cu") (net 10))
 (segment (start 139.6111 119.6086) (end 145.9611 119.6086) (width 1.27) (layer "B.Cu") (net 11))
 (segment (start 139.6111 119.8786) (end 139.6111 119.6086) (width 1.27) (layer "B.Cu") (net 11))
 (segment (start 145.9611 119.6086) (end 145.9611 118.3386) (width 1.27) (layer "B.Cu") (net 11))
 (segment (start 161.2011 120.8786) (end 161.2011 118.3386) (width 1.27) (layer "B.Cu") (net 16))
 (segment (start 153.1211 121.3386) (end 153.5811 120.8786) (width 1.27) (layer "B.Cu") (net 16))
 (segment (start 153.5811 120.8786) (end 161.2011 120.8786) (width 1.27) (layer "B.Cu") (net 16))
 (segment (start 153.1211 123.4186) (end 153.1211 121.3386) (width 1.27) (layer "B.Cu") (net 16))
 (segment (start 161.2011 115.7986) (end 154.8511 122.1486) (width 1.27) (layer "F.Cu") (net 17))
 (segment (start 154.8511 122.1486) (end 154.8511 123.1486) (width 1.27) (layer "F.Cu") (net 17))
 (segment (start 154.8511 123.1486) (end 155.1211 123.4186) (width 1.27) (layer "F.Cu") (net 17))
 (segment (start 168.14775 120.9642) (end 166.2811 120.8786) (width 0.8128) (layer "B.Cu") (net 12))
 (segment (start 168.8211 121.3386) (end 168.14775 120.9642) (width 0.8128) (layer "B.Cu") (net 12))
 (segment (start 166.2811 120.8786) (end 162.4711 114.5286) (width 0.8128) (layer "B.Cu") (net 12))
 (segment (start 162.4711 114.5286) (end 161.2011 113.2586) (width 0.8128) (layer "B.Cu") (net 12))
 (segment (start 164.6441 113.2586) (end 162.9226 111.5371) (width 1.27) (layer "B.Cu") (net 13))
 (segment (start 166.2811 113.2586) (end 164.6441 113.2586) (width 1.27) (layer "B.Cu") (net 13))
 (segment (start 166.4335 115.6462) (end 166.2811 115.6462) (width 1.27) (layer "B.Cu") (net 13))
 (segment (start 167.4335 119.3386) (end 166.4335 118.3386) (width 1.27) (layer "B.Cu") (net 13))
 (segment (start 166.4335 118.3386) (end 166.4335 115.6462) (width 1.27) (layer "B.Cu") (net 13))
 (segment (start 168.8211 119.3386) (end 167.4335 119.3386) (width 1.27) (layer "B.Cu") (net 13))
 (segment (start 166.2811 115.6462) (end 166.2811 113.2586) (width 1.27) (layer "B.Cu") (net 13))
 (segment (start 162.9226 111.5371) (end 162.4711 111.5371) (width 1.27) (layer "B.Cu") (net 13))
 (segment (start 162.4711 111.5371) (end 162.4711 110.7186) (width 1.27) (layer "B.Cu") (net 13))
 (segment (start 162.4711 110.7186) (end 161.2011 110.7186) (width 1.27) (layer "B.Cu") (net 13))
 (segment (start 161.2011 108.9971) (end 161.2011 108.1786) (width 1.27) (layer "B.Cu") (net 6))
 (segment (start 168.8211 111.1786) (end 165.0111 111.1786) (width 1.27) (layer "B.Cu") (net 6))
 (segment (start 165.0111 108.9971) (end 161.2011 108.9971) (width 1.27) (layer "B.Cu") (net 6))
 (segment (start 165.0111 111.1786) (end 165.0111 108.9971) (width 1.27) (layer "B.Cu") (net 6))
 (segment (start 167.0939 109.4486) (end 167.0939 105.6386) (width 1.27) (layer "B.Cu") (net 7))
 (segment (start 168.8211 109.1786) (end 168.8211 109.4486) (width 1.27) (layer "B.Cu") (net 7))
 (segment (start 168.8211 109.4486) (end 167.0939 109.4486) (width 1.27) (layer "B.Cu") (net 7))
 (segment (start 167.0939 105.6386) (end 161.2011 105.6386) (width 1.27) (layer "B.Cu") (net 7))
 (segment (start 168.8211 103.0986) (end 161.2011 103.0986) (width 1.27) (layer "B.Cu") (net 8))
 (segment (start 168.8211 101.0186) (end 168.8211 103.0986) (width 1.27) (layer "B.Cu") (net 8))
 (segment (start 168.8211 99.0186) (end 168.8211 99.2914) (width 1.27) (layer "B.Cu") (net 9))
 (segment (start 168.8211 99.2914) (end 167.0939 99.2914) (width 1.27) (layer "B.Cu") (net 9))
 (segment (start 167.0939 99.2914) (end 167.0939 100.5586) (width 1.27) (layer "B.Cu") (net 9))
 (segment (start 167.0939 100.5586) (end 161.2011 100.5586) (width 1.27) (layer "B.Cu") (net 9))
 (segment (start 167.0939 96.7486) (end 165.0111 96.7486) (width 1.27) (layer "B.Cu") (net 18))
 (segment (start 168.8211 90.8586) (end 168.8211 93.2914) (width 1.27) (layer "B.Cu") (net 18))
 (segment (start 167.0939 93.2914) (end 167.0939 96.7486) (width 1.27) (layer "B.Cu") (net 18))
 (segment (start 165.0111 96.7486) (end 165.0111 98.0186) (width 1.27) (layer "B.Cu") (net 18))
 (segment (start 165.0111 98.0186) (end 161.2011 98.0186) (width 1.27) (layer "B.Cu") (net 18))
 (segment (start 168.8211 93.2914) (end 167.0939 93.2914) (width 1.27) (layer "B.Cu") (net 18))
 (segment (start 166.2811 91.6686) (end 166.2811 90.3986) (width 1.27) (layer "B.Cu") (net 19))
 (segment (start 167.8211 88.8586) (end 168.8211 88.8586) (width 1.27) (layer "B.Cu") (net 19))
 (segment (start 161.2011 95.4786) (end 166.2811 91.6686) (width 0.8128) (layer "B.Cu") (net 19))
 (segment (start 166.2811 90.3986) (end 167.8211 88.8586) (width 1.27) (layer "B.Cu") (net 19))
 (segment (start 163.7411 85.3186) (end 159.1211 85.3186) (width 1.27) (layer "B.Cu") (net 22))
 (segment (start 161.2011 92.9386) (end 163.7411 90.3986) (width 1.27) (layer "B.Cu") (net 22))
 (segment (start 163.7411 90.3986) (end 163.7411 85.3186) (width 1.27) (layer "B.Cu") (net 22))
 (segment (start 157.1211 90.1286) (end 157.1211 85.3186) (width 1.27) (layer "B.Cu") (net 23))
 (segment (start 157.3911 90.3986) (end 157.1211 90.1286) (width 1.27) (layer "B.Cu") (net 23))
 (segment (start 161.2011 90.3986) (end 157.3911 90.3986) (width 1.27) (layer "B.Cu") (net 23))
 (segment (start 134.5311 122.1486) (end 134.5311 123.4186) (width 1.27) (layer "B.Cu") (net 1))
 (segment (start 150.956434 87.8586) (end 153.5811 87.8586) (width 1.27) (layer "B.Cu") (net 1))
 (segment (start 153.5811 87.8586) (end 155.1211 86.3186) (width 1.27) (layer "B.Cu") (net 1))
 (segment (start 150.7871 126.2126) (end 135.2423 126.2126) (width 1.27) (layer "B.Cu") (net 1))
 (segment (start 168.8211 117.3386) (end 170.9039 117.3386) (width 1.27) (layer "B.Cu") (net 1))
 (segment (start 150.7871 90.3986) (end 150.956434 87.8586) (width 1.27) (layer "B.Cu") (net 1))
 (segment (start 134.5311 111.7186) (end 134.5311 122.1486) (width 1.27) (layer "B.Cu") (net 1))
 (segment (start 139.6111 122.1486) (end 134.5311 122.1486) (width 1.27) (layer "B.Cu") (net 1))
 (segment (start 168.8211 97.0186) (end 170.9039 97.0186) (width 1.27) (layer "B.Cu") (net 1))
 (segment (start 157.1211 125.6886) (end 157.3911 125.9586) (width 1.27) (layer "B.Cu") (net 1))
 (segment (start 170.9039 97.0186) (end 170.9039 86.8586) (width 1.27) (layer "B.Cu") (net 1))
 (segment (start 157.1211 123.4186) (end 157.1211 125.6886) (width 1.27) (layer "B.Cu") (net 1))
 (segment (start 170.9039 86.8586) (end 168.8211 86.8586) (width 1.27) (layer "B.Cu") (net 1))
 (segment (start 129.4511 123.3786) (end 129.4911 123.4186) (width 1.27) (layer "B.Cu") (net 1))
 (segment (start 129.4911 123.4186) (end 134.5311 123.4186) (width 1.27) (layer "B.Cu") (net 1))
 (segment (start 155.1211 86.3186) (end 155.1211 85.3186) (width 1.27) (layer "B.Cu") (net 1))
 (segment (start 135.2423 126.2126) (end 134.5311 125.5014) (width 1.27) (layer "B.Cu") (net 1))
 (segment (start 170.9039 125.9586) (end 170.9039 117.3386) (width 1.27) (layer "B.Cu") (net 1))
 (segment (start 168.8211 107.1786) (end 170.9039 107.1786) (width 1.27) (layer "B.Cu") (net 1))
 (segment (start 139.6111 111.7186) (end 134.5311 111.7186) (width 1.27) (layer "B.Cu") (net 1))
 (segment (start 145.9611 90.3986) (end 139.6911 90.3986) (width 1.27) (layer "B.Cu") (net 1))
 (segment (start 157.3911 125.9586) (end 170.9039 125.9586) (width 1.27) (layer "B.Cu") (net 1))
 (segment (start 139.6111 121.8786) (end 139.6111 122.1486) (width 1.27) (layer "B.Cu") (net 1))
 (segment (start 139.6911 90.3986) (end 139.6111 90.4786) (width 1.27) (layer "B.Cu") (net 1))
 (segment (start 170.9039 117.3386) (end 170.9039 107.1786) (width 1.27) (layer "B.Cu") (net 1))
 (segment (start 150.7871 126.2126) (end 150.7871 90.3986) (width 1.27) (layer "B.Cu") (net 1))
 (segment (start 170.9039 107.1786) (end 170.9039 97.0186) (width 1.27) (layer "B.Cu") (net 1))
 (segment (start 150.7871 126.2126) (end 157.1371 126.2126) (width 1.27) (layer "B.Cu") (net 1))
 (segment (start 134.5311 123.4186) (end 134.5311 125.5014) (width 1.27) (layer "B.Cu") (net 1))
 (segment (start 145.9611 90.3986) (end 150.7871 90.3986) (width 1.27) (layer "B.Cu") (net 1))
 (segment (start 157.1371 126.2126) (end 157.3911 125.9586) (width 1.27) (layer "B.Cu") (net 1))
 (segment (start 165.0111 87.8586) (end 165.0111 84.8586) (width 1.27) (layer "F.Cu") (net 2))
 (segment (start 148.0439 125.9586) (end 148.5011 125.5014) (width 1.27) (layer "F.Cu") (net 2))
 (segment (start 140.37005 92.9386) (end 140.28445 92.853) (width 1.27) (layer "F.Cu") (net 2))
 (segment (start 165.0111 123.4186) (end 159.1211 123.4186) (width 1.27) (layer "F.Cu") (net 2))
 (segment (start 129.4111 110.7186) (end 126.0983 110.7186) (width 1.27) (layer "F.Cu") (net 2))
 (segment (start 168.8211 84.8586) (end 165.0111 84.8586) (width 1.27) (layer "F.Cu") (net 2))
 (segment (start 165.0111 115.3386) (end 165.0111 123.4186) (width 1.27) (layer "F.Cu") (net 2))
 (segment (start 148.5853 126.5) (end 165.5 126.5) (width 1.27) (layer "F.Cu") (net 2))
 (segment (start 165.0111 105.1786) (end 165.0111 95.0186) (width 1.27) (layer "F.Cu") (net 2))
 (segment (start 145.9611 92.9386) (end 148.5011 92.9386) (width 1.27) (layer "F.Cu") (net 2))
 (segment (start 165.5 126.5) (end 165.5 123.9075) (width 1.27) (layer "F.Cu") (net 2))
 (segment (start 137.0711 125.9586) (end 148.0439 125.9586) (width 1.27) (layer "F.Cu") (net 2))
 (segment (start 139.6111 113.7186) (end 137.0711 113.7186) (width 1.27) (layer "F.Cu") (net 2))
 (segment (start 139.6111 123.8786) (end 137.1925 123.8786) (width 1) (layer "F.Cu") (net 2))
 (segment (start 165.0111 95.0186) (end 165.0111 87.8586) (width 1.27) (layer "F.Cu") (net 2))
 (segment (start 137.0711 124) (end 137.0711 125.9586) (width 1.27) (layer "F.Cu") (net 2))
 (segment (start 168.8211 105.1786) (end 165.0111 105.1786) (width 1.27) (layer "F.Cu") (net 2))
 (segment (start 126.0983 94.2086) (end 129.4511 94.2086) (width 1.27) (layer "F.Cu") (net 2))
 (segment (start 137.0711 118.3386) (end 137.0711 124) (width 1.27) (layer "F.Cu") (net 2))
 (segment (start 126.0983 110.7186) (end 126.0983 94.2086) (width 1.27) (layer "F.Cu") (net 2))
 (segment (start 168.8211 95.0186) (end 165.0111 95.0186) (width 1.27) (layer "F.Cu") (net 2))
 (segment (start 140.28445 92.853) (end 139.6111 92.853) (width 1.27) (layer "F.Cu") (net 2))
 (segment (start 129.4511 110.6786) (end 129.4511 118.3386) (width 1.27) (layer "F.Cu") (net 2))
 (segment (start 165.5 123.9075) (end 165.0111 123.4186) (width 1.27) (layer "F.Cu") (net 2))
 (segment (start 148.5011 95.4786) (end 148.5011 92.9386) (width 1.27) (layer "F.Cu") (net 2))
 (segment (start 148.5011 95.4786) (end 158.6611 95.4786) (width 1.27) (layer "F.Cu") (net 2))
 (segment (start 158.6611 87.8586) (end 165.0111 87.8586) (width 1.27) (layer "F.Cu") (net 2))
 (segment (start 148.5011 92.9386) (end 148.5011 85.3186) (width 1.27) (layer "F.Cu") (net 2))
 (segment (start 137.0711 113.7186) (end 137.0711 118.3386) (width 1.27) (layer "F.Cu") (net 2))
 (segment (start 148.5011 125.5014) (end 148.5011 95.4786) (width 1.27) (layer "F.Cu") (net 2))
 (segment (start 129.4911 118.3386) (end 137.0711 118.3386) (width 1.27) (layer "F.Cu") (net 2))
 (segment (start 145.9611 92.9386) (end 140.37005 92.9386) (width 1.27) (layer "F.Cu") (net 2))
 (segment (start 148.5011 85.3186) (end 153.1211 85.3186) (width 1.27) (layer "F.Cu") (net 2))
 (segment (start 165.0111 105.1786) (end 165.0111 115.3386) (width 1.27) (layer "F.Cu") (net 2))
 (segment (start 148.0439 125.9586) (end 148.5853 126.5) (width 1.27) (layer "F.Cu") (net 2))
 (segment (start 137.1925 123.8786) (end 137.0711 124) (width 1) (layer "F.Cu") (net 2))
 (segment (start 129.4511 110.6786) (end 129.4111 110.7186) (width 1.27) (layer "F.Cu") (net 2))
 (segment (start 168.8211 115.3386) (end 165.0111 115.3386) (width 1.27) (layer "F.Cu") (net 2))
 (segment (start 158.6611 95.4786) (end 158.6611 87.8586) (width 1.27) (layer "F.Cu") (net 2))
 (segment (start 129.4511 118.3786) (end 129.4911 118.3386) (width 1.27) (layer "F.Cu") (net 2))
 (segment (start 142.1511 103.0986) (end 139.6111 100.5586) (width 1.27) (layer "B.Cu") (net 5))
 (segment (start 139.6111 100.5586) (end 139.6111 98.4786) (width 1.27) (layer "B.Cu") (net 5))
 (segment (start 134.5311 96.7486) (end 134.5311 103.0986) (width 1.27) (layer "B.Cu") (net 14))
 (segment (start 129.4511 96.7486) (end 134.5311 96.7486) (width 1.27) (layer "B.Cu") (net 14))
 (segment (start 129.4511 105.6786) (end 129.4511 99.2886) (width 1.27) (layer "F.Cu") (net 15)))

